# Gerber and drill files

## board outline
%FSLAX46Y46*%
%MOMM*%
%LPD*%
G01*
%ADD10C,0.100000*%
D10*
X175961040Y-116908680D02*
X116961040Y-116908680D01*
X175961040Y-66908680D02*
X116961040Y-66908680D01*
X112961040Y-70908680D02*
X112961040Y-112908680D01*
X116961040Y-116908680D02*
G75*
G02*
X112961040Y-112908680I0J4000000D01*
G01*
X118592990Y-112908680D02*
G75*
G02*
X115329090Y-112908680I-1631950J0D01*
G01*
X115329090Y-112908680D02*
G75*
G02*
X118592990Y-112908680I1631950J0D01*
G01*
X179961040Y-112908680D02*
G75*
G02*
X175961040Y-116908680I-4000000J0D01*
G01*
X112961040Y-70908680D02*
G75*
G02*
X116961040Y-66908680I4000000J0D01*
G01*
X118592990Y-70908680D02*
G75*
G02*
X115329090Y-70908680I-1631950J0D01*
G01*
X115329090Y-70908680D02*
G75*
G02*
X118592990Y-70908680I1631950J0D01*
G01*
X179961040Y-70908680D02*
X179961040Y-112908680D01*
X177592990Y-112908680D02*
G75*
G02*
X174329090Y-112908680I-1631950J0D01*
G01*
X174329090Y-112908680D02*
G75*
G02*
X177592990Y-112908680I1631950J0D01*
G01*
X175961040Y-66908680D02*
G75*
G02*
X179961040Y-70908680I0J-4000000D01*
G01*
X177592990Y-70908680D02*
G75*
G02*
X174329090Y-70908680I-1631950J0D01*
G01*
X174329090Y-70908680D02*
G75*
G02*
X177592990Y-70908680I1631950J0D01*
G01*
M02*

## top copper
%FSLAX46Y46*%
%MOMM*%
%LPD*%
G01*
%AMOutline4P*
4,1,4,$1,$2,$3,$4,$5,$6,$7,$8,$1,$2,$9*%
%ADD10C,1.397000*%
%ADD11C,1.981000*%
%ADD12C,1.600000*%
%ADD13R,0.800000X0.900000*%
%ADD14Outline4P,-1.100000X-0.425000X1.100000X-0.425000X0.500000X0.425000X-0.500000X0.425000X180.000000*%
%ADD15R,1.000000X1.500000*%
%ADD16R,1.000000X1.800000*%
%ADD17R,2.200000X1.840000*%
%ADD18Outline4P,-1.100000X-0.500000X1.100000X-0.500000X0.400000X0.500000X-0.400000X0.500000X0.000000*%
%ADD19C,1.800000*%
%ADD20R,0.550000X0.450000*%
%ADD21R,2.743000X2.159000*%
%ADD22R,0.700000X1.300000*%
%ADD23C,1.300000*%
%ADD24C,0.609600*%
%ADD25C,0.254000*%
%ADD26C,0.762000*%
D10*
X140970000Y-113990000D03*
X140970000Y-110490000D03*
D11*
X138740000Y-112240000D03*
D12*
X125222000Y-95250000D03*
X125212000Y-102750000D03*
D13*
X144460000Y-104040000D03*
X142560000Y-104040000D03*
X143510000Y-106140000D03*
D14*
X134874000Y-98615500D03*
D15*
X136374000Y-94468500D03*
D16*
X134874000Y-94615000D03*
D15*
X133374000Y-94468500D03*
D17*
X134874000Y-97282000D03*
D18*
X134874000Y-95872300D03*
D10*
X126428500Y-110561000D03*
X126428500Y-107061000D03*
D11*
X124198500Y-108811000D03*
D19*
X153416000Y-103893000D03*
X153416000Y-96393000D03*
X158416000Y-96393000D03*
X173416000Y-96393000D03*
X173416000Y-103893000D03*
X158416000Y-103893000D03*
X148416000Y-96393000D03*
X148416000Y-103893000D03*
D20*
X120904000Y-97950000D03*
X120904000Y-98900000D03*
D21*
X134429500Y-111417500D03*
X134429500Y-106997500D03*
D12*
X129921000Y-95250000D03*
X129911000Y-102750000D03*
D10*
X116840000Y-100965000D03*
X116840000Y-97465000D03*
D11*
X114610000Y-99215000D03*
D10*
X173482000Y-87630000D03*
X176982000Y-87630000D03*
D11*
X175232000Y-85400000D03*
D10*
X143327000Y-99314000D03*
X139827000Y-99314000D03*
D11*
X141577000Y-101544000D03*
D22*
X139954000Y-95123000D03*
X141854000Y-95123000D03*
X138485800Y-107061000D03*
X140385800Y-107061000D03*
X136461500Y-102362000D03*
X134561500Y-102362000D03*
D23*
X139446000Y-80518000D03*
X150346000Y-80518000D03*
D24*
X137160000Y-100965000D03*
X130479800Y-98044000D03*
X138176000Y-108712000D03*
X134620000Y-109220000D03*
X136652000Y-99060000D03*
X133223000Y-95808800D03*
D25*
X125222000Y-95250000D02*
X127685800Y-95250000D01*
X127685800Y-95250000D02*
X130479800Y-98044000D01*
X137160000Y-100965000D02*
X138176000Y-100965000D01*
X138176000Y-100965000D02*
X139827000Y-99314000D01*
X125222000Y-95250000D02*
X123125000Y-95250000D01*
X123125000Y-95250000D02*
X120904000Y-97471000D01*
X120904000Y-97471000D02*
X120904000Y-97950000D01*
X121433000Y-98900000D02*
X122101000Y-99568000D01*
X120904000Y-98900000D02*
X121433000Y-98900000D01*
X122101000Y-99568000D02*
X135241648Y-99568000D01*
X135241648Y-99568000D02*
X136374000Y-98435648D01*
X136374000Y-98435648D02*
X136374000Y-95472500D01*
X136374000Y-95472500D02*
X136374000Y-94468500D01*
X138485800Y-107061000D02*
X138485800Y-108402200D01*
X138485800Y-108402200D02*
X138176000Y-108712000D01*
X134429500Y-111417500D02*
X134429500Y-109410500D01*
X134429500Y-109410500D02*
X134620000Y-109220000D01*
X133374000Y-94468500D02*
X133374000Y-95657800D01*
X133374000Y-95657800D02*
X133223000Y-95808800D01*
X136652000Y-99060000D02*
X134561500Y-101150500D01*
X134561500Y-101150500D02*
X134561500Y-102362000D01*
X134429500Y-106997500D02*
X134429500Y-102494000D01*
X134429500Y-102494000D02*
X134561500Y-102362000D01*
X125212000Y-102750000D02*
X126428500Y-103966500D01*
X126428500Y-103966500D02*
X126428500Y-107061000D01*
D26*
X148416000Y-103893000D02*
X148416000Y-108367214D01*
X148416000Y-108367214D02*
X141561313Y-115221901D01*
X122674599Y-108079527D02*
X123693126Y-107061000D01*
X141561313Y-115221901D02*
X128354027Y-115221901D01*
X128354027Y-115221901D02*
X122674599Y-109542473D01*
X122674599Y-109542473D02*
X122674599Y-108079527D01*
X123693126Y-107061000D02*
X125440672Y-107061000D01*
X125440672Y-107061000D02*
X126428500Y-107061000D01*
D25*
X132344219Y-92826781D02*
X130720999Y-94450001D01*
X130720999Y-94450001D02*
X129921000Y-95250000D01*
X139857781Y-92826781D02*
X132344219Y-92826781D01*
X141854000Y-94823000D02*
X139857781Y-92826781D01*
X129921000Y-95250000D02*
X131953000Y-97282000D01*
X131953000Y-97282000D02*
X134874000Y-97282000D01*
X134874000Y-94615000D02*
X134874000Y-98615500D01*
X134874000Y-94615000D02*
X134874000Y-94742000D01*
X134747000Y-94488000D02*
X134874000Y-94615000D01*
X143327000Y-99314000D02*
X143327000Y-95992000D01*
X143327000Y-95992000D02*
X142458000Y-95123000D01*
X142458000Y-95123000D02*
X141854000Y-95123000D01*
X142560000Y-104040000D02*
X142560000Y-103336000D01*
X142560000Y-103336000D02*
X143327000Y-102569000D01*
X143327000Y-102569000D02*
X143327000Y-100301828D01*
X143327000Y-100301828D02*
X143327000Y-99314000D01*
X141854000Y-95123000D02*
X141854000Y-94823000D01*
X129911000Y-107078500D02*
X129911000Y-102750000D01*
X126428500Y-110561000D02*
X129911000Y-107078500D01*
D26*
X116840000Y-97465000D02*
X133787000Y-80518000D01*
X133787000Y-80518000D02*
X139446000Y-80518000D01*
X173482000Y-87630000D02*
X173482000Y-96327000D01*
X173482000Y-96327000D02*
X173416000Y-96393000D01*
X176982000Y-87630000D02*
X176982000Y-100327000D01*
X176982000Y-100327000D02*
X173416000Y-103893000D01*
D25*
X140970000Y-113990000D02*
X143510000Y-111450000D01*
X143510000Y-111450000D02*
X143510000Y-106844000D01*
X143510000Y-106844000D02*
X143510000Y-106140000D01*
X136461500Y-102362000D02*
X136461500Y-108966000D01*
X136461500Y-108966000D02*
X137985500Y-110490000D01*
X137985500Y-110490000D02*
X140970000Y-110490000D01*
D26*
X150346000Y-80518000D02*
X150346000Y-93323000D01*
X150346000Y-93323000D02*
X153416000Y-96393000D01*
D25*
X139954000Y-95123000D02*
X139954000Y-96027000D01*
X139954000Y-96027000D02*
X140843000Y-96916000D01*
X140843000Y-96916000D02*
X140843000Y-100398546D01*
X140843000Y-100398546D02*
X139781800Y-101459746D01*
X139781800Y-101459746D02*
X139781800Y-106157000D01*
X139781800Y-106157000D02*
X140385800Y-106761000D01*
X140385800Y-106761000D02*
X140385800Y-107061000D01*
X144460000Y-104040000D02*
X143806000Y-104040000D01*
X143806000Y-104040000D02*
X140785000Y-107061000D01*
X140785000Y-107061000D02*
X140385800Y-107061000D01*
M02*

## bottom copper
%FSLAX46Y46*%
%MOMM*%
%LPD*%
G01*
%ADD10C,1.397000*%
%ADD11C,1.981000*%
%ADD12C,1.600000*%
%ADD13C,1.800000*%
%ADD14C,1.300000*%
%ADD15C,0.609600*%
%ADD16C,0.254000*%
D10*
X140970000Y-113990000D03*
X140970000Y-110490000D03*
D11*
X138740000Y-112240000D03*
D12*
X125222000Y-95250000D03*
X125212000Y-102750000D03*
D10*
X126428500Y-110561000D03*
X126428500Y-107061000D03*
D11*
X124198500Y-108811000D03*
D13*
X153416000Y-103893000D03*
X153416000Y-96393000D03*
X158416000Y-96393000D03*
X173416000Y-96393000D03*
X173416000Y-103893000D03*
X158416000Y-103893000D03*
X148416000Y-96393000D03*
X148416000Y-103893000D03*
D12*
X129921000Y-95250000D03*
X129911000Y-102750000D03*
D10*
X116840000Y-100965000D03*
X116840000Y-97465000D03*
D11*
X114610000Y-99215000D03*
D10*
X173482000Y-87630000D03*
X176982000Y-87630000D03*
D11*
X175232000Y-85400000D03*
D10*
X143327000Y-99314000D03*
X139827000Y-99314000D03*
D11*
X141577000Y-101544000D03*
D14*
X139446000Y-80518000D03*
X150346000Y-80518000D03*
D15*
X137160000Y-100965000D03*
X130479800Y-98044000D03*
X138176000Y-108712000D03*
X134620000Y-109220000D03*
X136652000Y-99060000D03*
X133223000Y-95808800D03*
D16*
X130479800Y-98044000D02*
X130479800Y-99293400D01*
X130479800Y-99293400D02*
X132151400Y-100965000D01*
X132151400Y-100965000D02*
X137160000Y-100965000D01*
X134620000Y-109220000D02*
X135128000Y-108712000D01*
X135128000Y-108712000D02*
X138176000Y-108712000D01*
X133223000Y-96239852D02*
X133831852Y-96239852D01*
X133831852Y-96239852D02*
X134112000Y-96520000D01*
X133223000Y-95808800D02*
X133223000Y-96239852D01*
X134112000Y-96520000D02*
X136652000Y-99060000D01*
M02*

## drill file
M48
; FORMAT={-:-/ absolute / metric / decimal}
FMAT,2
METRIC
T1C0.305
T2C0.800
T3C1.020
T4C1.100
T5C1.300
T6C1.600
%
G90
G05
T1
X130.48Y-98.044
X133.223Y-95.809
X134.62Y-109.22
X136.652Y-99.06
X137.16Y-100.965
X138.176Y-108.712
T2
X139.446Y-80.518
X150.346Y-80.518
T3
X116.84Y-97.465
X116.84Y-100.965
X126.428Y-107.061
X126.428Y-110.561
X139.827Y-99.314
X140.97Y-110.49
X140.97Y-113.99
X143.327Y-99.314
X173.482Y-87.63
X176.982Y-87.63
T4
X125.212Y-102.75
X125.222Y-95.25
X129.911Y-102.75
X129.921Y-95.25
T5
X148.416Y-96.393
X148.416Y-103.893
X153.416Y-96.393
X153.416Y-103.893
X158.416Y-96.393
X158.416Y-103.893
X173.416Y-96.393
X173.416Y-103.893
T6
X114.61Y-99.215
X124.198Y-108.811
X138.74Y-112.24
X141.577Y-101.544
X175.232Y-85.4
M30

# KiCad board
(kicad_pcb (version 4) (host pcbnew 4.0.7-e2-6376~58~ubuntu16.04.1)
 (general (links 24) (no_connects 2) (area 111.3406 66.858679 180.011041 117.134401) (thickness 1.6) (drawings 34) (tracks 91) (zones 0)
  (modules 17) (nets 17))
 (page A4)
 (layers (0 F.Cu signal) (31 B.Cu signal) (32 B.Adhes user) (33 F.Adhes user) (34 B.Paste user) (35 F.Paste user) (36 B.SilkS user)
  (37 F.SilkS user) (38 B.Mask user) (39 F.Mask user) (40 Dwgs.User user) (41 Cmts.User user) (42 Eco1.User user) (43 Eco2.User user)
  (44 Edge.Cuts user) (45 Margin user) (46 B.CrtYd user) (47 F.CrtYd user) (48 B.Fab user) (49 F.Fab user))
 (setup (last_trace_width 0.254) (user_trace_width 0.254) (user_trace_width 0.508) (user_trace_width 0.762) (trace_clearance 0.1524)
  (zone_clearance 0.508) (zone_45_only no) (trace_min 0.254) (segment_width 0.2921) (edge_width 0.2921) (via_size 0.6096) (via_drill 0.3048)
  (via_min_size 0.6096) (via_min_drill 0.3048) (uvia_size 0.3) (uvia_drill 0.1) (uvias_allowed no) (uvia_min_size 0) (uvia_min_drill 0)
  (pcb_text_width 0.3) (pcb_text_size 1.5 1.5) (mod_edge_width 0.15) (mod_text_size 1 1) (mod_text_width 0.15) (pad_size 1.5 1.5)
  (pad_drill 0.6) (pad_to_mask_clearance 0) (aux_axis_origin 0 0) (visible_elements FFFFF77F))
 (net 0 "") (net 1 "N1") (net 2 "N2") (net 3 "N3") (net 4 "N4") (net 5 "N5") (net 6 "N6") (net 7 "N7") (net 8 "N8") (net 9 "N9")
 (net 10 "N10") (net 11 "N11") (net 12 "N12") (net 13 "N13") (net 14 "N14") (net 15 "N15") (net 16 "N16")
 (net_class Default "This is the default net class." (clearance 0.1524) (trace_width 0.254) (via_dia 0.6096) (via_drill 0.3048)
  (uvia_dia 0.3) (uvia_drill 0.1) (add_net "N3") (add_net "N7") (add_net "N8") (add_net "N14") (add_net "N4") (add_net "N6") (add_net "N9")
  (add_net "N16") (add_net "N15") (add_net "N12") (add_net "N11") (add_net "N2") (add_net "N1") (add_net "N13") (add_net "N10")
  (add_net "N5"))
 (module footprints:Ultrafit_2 (layer F.Cu) (at 140.97 113.99 180)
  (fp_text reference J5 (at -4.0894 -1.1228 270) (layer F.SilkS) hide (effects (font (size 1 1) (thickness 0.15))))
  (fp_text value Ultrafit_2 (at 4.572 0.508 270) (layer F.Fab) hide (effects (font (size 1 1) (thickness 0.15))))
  (pad 2 thru_hole circle (at 0 0 180) (size 1.397 1.397) (drill 1.02) (layers *.Cu *.Mask) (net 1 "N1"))
  (pad 1 thru_hole circle (at 0 3.5 180) (size 1.397 1.397) (drill 1.02) (layers *.Cu *.Mask) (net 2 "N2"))
  (pad "" thru_hole circle (at 2.23 1.75 180) (size 1.981 1.981) (drill 1.6) (layers *.Cu *.Mask)))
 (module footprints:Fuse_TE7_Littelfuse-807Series (layer F.Cu) (at 125.222 95.25 270)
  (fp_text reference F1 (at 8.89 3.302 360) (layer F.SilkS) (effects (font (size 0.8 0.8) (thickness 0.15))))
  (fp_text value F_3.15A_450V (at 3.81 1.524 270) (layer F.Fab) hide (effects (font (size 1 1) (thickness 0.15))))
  (pad 1 thru_hole circle (at 0 0 270) (size 1.6 1.6) (drill 1.1) (layers *.Cu *.Mask) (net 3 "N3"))
  (pad 2 thru_hole circle (at 7.5 0.01 270) (size 1.6 1.6) (drill 1.1) (layers *.Cu *.Mask) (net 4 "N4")))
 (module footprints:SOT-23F (layer F.Cu) (at 143.51 105.09 270)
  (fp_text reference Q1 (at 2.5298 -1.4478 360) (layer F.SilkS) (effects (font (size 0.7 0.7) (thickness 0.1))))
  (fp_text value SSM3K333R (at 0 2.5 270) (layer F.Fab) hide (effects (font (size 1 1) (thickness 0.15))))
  (pad 1 smd rect (at -1.05 -0.95 270) (size 0.9 0.8) (layers F.Cu F.Paste F.Mask) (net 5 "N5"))
  (pad 2 smd rect (at -1.05 0.95 270) (size 0.9 0.8) (layers F.Cu F.Paste F.Mask) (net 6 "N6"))
  (pad 3 smd rect (at 1.05 0 270) (size 0.9 0.8) (layers F.Cu F.Paste F.Mask) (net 1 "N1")))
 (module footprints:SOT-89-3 (layer F.Cu) (at 134.874 95.9485 270)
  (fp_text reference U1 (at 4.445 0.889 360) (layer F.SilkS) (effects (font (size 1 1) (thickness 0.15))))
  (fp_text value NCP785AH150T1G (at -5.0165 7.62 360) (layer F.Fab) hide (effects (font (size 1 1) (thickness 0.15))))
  (pad 2 smd trapezoid (at 2.667 0 180) (size 1.6 0.85) (rect_delta 0 0.6) (layers F.Cu F.Paste F.Mask) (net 6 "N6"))
  (pad 1 smd rect (at -1.48 -1.5 180) (size 1 1.5) (layers F.Cu F.Paste F.Mask) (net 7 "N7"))
  (pad 2 smd rect (at -1.3335 0 180) (size 1 1.8) (layers F.Cu F.Paste F.Mask) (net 6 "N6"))
  (pad 3 smd rect (at -1.48 1.5 180) (size 1 1.5) (layers F.Cu F.Paste F.Mask) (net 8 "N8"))
  (pad 2 smd rect (at 1.3335 0 180) (size 2.2 1.84) (layers F.Cu F.Paste F.Mask) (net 6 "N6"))
  (pad 2 smd trapezoid (at -0.0762 0) (size 1.5 1) (rect_delta 0 0.7) (layers F.Cu F.Paste F.Mask) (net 6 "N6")))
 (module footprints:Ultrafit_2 (layer F.Cu) (at 126.4285 110.561 180)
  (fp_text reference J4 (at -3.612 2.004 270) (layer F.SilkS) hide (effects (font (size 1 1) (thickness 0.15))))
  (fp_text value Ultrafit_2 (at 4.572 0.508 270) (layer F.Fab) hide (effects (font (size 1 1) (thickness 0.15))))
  (pad 2 thru_hole circle (at 0 0 180) (size 1.397 1.397) (drill 1.02) (layers *.Cu *.Mask) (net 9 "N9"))
  (pad 1 thru_hole circle (at 0 3.5 180) (size 1.397 1.397) (drill 1.02) (layers *.Cu *.Mask) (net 4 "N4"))
  (pad "" thru_hole circle (at 2.23 1.75 180) (size 1.981 1.981) (drill 1.6) (layers *.Cu *.Mask)))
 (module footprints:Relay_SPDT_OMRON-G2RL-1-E (layer F.Cu) (at 173.416 96.393 180)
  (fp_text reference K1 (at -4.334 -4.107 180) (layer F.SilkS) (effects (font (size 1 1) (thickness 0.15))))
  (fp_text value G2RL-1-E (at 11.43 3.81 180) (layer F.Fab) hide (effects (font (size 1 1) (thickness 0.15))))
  (pad 3 thru_hole circle (at 20 -7.5 180) (size 1.8 1.8) (drill 1.3) (layers *.Cu *.Mask))
  (pad 6 thru_hole circle (at 20 0 180) (size 1.8 1.8) (drill 1.3) (layers *.Cu *.Mask) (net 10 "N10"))
  (pad 7 thru_hole circle (at 15 0 180) (size 1.8 1.8) (drill 1.3) (layers *.Cu *.Mask))
  (pad 8 thru_hole circle (at 0 0 180) (size 1.8 1.8) (drill 1.3) (layers *.Cu *.Mask) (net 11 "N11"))
  (pad 1 thru_hole circle (at 0 -7.5 180) (size 1.8 1.8) (drill 1.3) (layers *.Cu *.Mask) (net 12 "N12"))
  (pad 2 thru_hole circle (at 15 -7.5 180) (size 1.8 1.8) (drill 1.3) (layers *.Cu *.Mask) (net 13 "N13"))
  (pad 5 thru_hole circle (at 25 0 180) (size 1.8 1.8) (drill 1.3) (layers *.Cu *.Mask))
  (pad 4 thru_hole circle (at 25 -7.5 180) (size 1.8 1.8) (drill 1.3) (layers *.Cu *.Mask) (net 4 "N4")))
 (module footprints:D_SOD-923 (layer F.Cu) (at 120.904 98.425 270)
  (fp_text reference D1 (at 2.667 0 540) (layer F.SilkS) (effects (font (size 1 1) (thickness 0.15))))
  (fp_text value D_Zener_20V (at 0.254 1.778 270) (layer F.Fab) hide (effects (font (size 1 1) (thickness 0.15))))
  (pad 1 smd rect (at -0.475 0 270) (size 0.45 0.55) (layers F.Cu F.Paste F.Mask) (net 3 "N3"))
  (pad 2 smd rect (at 0.475 0 270) (size 0.45 0.55) (layers F.Cu F.Paste F.Mask) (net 7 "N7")))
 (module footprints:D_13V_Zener (layer F.Cu) (at 134.4295 109.2075 270)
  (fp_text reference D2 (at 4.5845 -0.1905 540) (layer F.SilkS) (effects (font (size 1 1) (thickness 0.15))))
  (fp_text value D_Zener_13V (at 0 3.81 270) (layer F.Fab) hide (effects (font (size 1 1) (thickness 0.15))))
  (pad 2 smd rect (at 2.21 0 90) (size 2.159 2.743) (layers F.Cu F.Paste F.Mask) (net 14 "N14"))
  (pad 1 smd rect (at -2.21 0 90) (size 2.159 2.743) (layers F.Cu F.Paste F.Mask) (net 8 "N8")))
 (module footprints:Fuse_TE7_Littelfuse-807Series (layer F.Cu) (at 129.921 95.25 270)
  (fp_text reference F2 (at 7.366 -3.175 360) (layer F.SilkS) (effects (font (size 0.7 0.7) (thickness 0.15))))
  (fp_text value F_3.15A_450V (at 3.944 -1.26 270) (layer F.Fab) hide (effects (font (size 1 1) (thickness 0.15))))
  (pad 1 thru_hole circle (at 0 0 270) (size 1.6 1.6) (drill 1.1) (layers *.Cu *.Mask) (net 6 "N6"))
  (pad 2 thru_hole circle (at 7.5 0.01 270) (size 1.6 1.6) (drill 1.1) (layers *.Cu *.Mask) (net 9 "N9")))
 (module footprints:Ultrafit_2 (layer F.Cu) (at 116.84 100.965 180)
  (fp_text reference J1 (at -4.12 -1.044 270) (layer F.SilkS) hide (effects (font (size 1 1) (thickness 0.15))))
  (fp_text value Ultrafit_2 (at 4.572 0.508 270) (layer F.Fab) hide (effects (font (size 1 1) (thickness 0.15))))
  (pad 2 thru_hole circle (at 0 0 180) (size 1.397 1.397) (drill 1.02) (layers *.Cu *.Mask) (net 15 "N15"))
  (pad 1 thru_hole circle (at 0 3.5 180) (size 1.397 1.397) (drill 1.02) (layers *.Cu *.Mask) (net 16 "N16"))
  (pad "" thru_hole circle (at 2.23 1.75 180) (size 1.981 1.981) (drill 1.6) (layers *.Cu *.Mask)))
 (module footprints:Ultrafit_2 (layer F.Cu) (at 173.482 87.63 90)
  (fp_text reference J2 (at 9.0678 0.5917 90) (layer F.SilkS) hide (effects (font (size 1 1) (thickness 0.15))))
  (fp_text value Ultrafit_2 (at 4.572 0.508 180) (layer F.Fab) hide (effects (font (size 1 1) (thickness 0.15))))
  (pad 2 thru_hole circle (at 0 0 90) (size 1.397 1.397) (drill 1.02) (layers *.Cu *.Mask) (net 11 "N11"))
  (pad 1 thru_hole circle (at 0 3.5 90) (size 1.397 1.397) (drill 1.02) (layers *.Cu *.Mask) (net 12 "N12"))
  (pad "" thru_hole circle (at 2.23 1.75 90) (size 1.981 1.981) (drill 1.6) (layers *.Cu *.Mask)))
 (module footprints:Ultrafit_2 (layer F.Cu) (at 143.327 99.314 270)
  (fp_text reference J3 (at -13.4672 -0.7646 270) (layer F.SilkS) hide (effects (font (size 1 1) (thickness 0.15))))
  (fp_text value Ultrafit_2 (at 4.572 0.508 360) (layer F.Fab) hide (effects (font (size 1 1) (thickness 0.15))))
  (pad 2 thru_hole circle (at 0 0 270) (size 1.397 1.397) (drill 1.02) (layers *.Cu *.Mask) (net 6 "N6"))
  (pad 1 thru_hole circle (at 0 3.5 270) (size 1.397 1.397) (drill 1.02) (layers *.Cu *.Mask) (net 3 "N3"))
  (pad "" thru_hole circle (at 2.23 1.75 270) (size 1.981 1.981) (drill 1.6) (layers *.Cu *.Mask)))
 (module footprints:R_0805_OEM (layer F.Cu) (at 140.904 95.123)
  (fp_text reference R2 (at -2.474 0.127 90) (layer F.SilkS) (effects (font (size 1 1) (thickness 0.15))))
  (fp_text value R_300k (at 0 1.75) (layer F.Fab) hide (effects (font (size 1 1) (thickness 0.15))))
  (pad 1 smd rect (at -0.95 0) (size 0.7 1.3) (layers F.Cu F.Paste F.Mask) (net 5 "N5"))
  (pad 2 smd rect (at 0.95 0) (size 0.7 1.3) (layers F.Cu F.Paste F.Mask) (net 6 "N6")))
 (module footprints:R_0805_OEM (layer F.Cu) (at 139.4358 107.061)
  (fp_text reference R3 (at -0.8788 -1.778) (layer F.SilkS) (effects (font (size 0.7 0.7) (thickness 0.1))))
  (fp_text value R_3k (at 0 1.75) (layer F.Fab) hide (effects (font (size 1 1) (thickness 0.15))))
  (pad 1 smd rect (at -0.95 0) (size 0.7 1.3) (layers F.Cu F.Paste F.Mask) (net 14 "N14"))
  (pad 2 smd rect (at 0.95 0) (size 0.7 1.3) (layers F.Cu F.Paste F.Mask) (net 5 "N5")))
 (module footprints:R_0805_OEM (layer F.Cu) (at 135.5115 102.362 180)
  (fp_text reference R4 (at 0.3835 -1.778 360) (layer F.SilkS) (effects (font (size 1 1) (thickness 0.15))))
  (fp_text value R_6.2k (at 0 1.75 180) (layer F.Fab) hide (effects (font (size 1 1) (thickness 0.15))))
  (pad 1 smd rect (at -0.95 0 180) (size 0.7 1.3) (layers F.Cu F.Paste F.Mask) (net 2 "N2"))
  (pad 2 smd rect (at 0.95 0 180) (size 0.7 1.3) (layers F.Cu F.Paste F.Mask) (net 8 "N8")))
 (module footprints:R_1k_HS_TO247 (layer F.Cu) (at 139.446 80.518)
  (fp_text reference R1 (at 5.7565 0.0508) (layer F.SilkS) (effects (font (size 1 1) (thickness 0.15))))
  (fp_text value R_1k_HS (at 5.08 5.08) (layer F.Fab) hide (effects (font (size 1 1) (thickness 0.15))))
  (pad 1 thru_hole circle (at 0 0) (size 1.3 1.3) (drill 0.8) (layers *.Cu *.Mask) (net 16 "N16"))
  (pad 2 thru_hole circle (at 10.9 0) (size 1.3 1.3) (drill 0.8) (layers *.Cu *.Mask) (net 10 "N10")))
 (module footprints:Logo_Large (layer B.Cu) (at 144.5895 73.2409 180)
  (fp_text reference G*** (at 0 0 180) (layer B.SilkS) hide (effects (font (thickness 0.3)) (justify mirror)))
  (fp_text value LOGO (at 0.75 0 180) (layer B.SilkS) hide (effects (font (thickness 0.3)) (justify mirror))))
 (gr_line (start 175.96104 116.90868) (end 116.96104 116.90868) (layer Edge.Cuts) (width 0.1))
 (gr_line (start 175.96104 66.90868) (end 116.96104 66.90868) (layer Edge.Cuts) (width 0.1))
 (gr_line (start 112.96104 70.90868) (end 112.96104 112.90868) (layer Edge.Cuts) (width 0.1))
 (gr_arc (start 116.96104 112.90868) (end 112.96104 112.90868) (angle -90) (layer Edge.Cuts) (width 0.1))
 (gr_circle (center 116.96104 112.90868) (end 118.59299 112.90868) (layer Edge.Cuts) (width 0.1))
 (gr_arc (start 175.96104 112.90868) (end 175.96104 116.90868) (angle -90) (layer Edge.Cuts) (width 0.1))
 (gr_arc (start 116.96104 70.90868) (end 116.96104 66.90868) (angle -90) (layer Edge.Cuts) (width 0.1))
 (gr_circle (center 116.96104 70.90868) (end 118.59299 70.90868) (layer Edge.Cuts) (width 0.1))
 (gr_line (start 179.96104 70.90868) (end 179.96104 112.90868) (layer Edge.Cuts) (width 0.1))
 (gr_circle (center 175.96104 112.90868) (end 177.59299 112.90868) (layer Edge.Cuts) (width 0.1))
 (gr_arc (start 175.96104 70.90868) (end 179.96104 70.90868) (angle -90) (layer Edge.Cuts) (width 0.1))
 (gr_circle (center 175.96104 70.90868) (end 177.59299 70.90868) (layer Edge.Cuts) (width 0.1))
 (segment (start 130.4798 98.044) (end 130.4798 99.2934) (width 0.254) (layer B.Cu) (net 3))
 (segment (start 130.4798 99.2934) (end 132.1514 100.965) (width 0.254) (layer B.Cu) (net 3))
 (segment (start 125.222 95.25) (end 127.6858 95.25) (width 0.254) (layer F.Cu) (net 3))
 (segment (start 127.6858 95.25) (end 130.4798 98.044) (width 0.254) (layer F.Cu) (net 3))
 (segment (start 137.16 100.965) (end 138.176 100.965) (width 0.254) (layer F.Cu) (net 3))
 (segment (start 138.176 100.965) (end 139.827 99.314) (width 0.254) (layer F.Cu) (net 3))
 (segment (start 132.1514 100.965) (end 137.16 100.965) (width 0.254) (layer B.Cu) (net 3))
 (via (at 137.16 100.965) (size 0.6096) (drill 0.3048) (layers F.Cu B.Cu) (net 3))
 (via (at 130.4798 98.044) (size 0.6096) (drill 0.3048) (layers F.Cu B.Cu) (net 3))
 (segment (start 125.222 95.25) (end 123.125 95.25) (width 0.254) (layer F.Cu) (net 3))
 (segment (start 123.125 95.25) (end 120.904 97.471) (width 0.254) (layer F.Cu) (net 3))
 (segment (start 120.904 97.471) (end 120.904 97.95) (width 0.254) (layer F.Cu) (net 3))
 (segment (start 121.433 98.9) (end 122.101 99.568) (width 0.254) (layer F.Cu) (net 7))
 (segment (start 120.904 98.9) (end 121.433 98.9) (width 0.254) (layer F.Cu) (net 7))
 (segment (start 122.101 99.568) (end 135.241648 99.568) (width 0.254) (layer F.Cu) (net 7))
 (segment (start 135.241648 99.568) (end 136.374 98.435648) (width 0.254) (layer F.Cu) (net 7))
 (segment (start 136.374 98.435648) (end 136.374 95.4725) (width 0.254) (layer F.Cu) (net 7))
 (segment (start 136.374 95.4725) (end 136.374 94.4685) (width 0.254) (layer F.Cu) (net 7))
 (segment (start 138.4858 107.061) (end 138.4858 108.4022) (width 0.254) (layer F.Cu) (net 14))
 (segment (start 138.4858 108.4022) (end 138.176 108.712) (width 0.254) (layer F.Cu) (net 14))
 (segment (start 134.62 109.22) (end 135.128 108.712) (width 0.254) (layer B.Cu) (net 14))
 (segment (start 135.128 108.712) (end 138.176 108.712) (width 0.254) (layer B.Cu) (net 14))
 (via (at 138.176 108.712) (size 0.6096) (drill 0.3048) (layers F.Cu B.Cu) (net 14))
 (segment (start 134.4295 111.4175) (end 134.4295 109.4105) (width 0.254) (layer F.Cu) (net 14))
 (segment (start 134.4295 109.4105) (end 134.62 109.22) (width 0.254) (layer F.Cu) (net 14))
 (via (at 134.62 109.22) (size 0.6096) (drill 0.3048) (layers F.Cu B.Cu) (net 14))
 (segment (start 133.374 94.4685) (end 133.374 95.6578) (width 0.254) (layer F.Cu) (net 8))
 (segment (start 133.374 95.6578) (end 133.223 95.8088) (width 0.254) (layer F.Cu) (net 8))
 (segment (start 133.223 96.239852) (end 133.831852 96.239852) (width 0.254) (layer B.Cu) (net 8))
 (segment (start 133.831852 96.239852) (end 134.112 96.52) (width 0.254) (layer B.Cu) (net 8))
 (segment (start 133.223 95.8088) (end 133.223 96.239852) (width 0.254) (layer B.Cu) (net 8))
 (segment (start 136.652 99.06) (end 134.5615 101.1505) (width 0.254) (layer F.Cu) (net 8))
 (segment (start 134.5615 101.1505) (end 134.5615 102.362) (width 0.254) (layer F.Cu) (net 8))
 (via (at 136.652 99.06) (size 0.6096) (drill 0.3048) (layers F.Cu B.Cu) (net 8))
 (segment (start 134.112 96.52) (end 136.652 99.06) (width 0.254) (layer B.Cu) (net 8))
 (via (at 133.223 95.8088) (size 0.6096) (drill 0.3048) (layers F.Cu B.Cu) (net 8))
 (segment (start 134.4295 106.9975) (end 134.4295 102.494) (width 0.254) (layer F.Cu) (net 8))
 (segment (start 134.4295 102.494) (end 134.5615 102.362) (width 0.254) (layer F.Cu) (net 8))
 (segment (start 125.212 102.75) (end 126.4285 103.9665) (width 0.254) (layer F.Cu) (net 4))
 (segment (start 126.4285 103.9665) (end 126.4285 107.061) (width 0.254) (layer F.Cu) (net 4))
 (segment (start 148.416 103.893) (end 148.416 108.367214) (width 0.762) (layer F.Cu) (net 4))
 (segment (start 148.416 108.367214) (end 141.561313 115.221901) (width 0.762) (layer F.Cu) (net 4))
 (segment (start 122.674599 108.079527) (end 123.693126 107.061) (width 0.762) (layer F.Cu) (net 4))
 (segment (start 141.561313 115.221901) (end 128.354027 115.221901) (width 0.762) (layer F.Cu) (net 4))
 (segment (start 128.354027 115.221901) (end 122.674599 109.542473) (width 0.762) (layer F.Cu) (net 4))
 (segment (start 122.674599 109.542473) (end 122.674599 108.079527) (width 0.762) (layer F.Cu) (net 4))
 (segment (start 123.693126 107.061) (end 125.440672 107.061) (width 0.762) (layer F.Cu) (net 4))
 (segment (start 125.440672 107.061) (end 126.4285 107.061) (width 0.762) (layer F.Cu) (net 4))
 (segment (start 132.344219 92.826781) (end 130.720999 94.450001) (width 0.254) (layer F.Cu) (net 6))
 (segment (start 130.720999 94.450001) (end 129.921 95.25) (width 0.254) (layer F.Cu) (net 6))
 (segment (start 139.857781 92.826781) (end 132.344219 92.826781) (width 0.254) (layer F.Cu) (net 6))
 (segment (start 141.854 94.823) (end 139.857781 92.826781) (width 0.254) (layer F.Cu) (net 6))
 (segment (start 129.921 95.25) (end 131.953 97.282) (width 0.254) (layer F.Cu) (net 6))
 (segment (start 131.953 97.282) (end 134.874 97.282) (width 0.254) (layer F.Cu) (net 6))
 (segment (start 134.874 94.615) (end 134.874 98.6155) (width 0.254) (layer F.Cu) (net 6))
 (segment (start 134.874 94.615) (end 134.874 94.742) (width 0.254) (layer F.Cu) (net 6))
 (segment (start 134.747 94.488) (end 134.874 94.615) (width 0.254) (layer F.Cu) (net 6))
 (segment (start 143.327 99.314) (end 143.327 95.992) (width 0.254) (layer F.Cu) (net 6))
 (segment (start 143.327 95.992) (end 142.458 95.123) (width 0.254) (layer F.Cu) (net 6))
 (segment (start 142.458 95.123) (end 141.854 95.123) (width 0.254) (layer F.Cu) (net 6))
 (segment (start 142.56 104.04) (end 142.56 103.336) (width 0.254) (layer F.Cu) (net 6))
 (segment (start 142.56 103.336) (end 143.327 102.569) (width 0.254) (layer F.Cu) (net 6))
 (segment (start 143.327 102.569) (end 143.327 100.301828) (width 0.254) (layer F.Cu) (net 6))
 (segment (start 143.327 100.301828) (end 143.327 99.314) (width 0.254) (layer F.Cu) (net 6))
 (segment (start 141.854 95.123) (end 141.854 94.823) (width 0.254) (layer F.Cu) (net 6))
 (segment (start 129.911 107.0785) (end 129.911 102.75) (width 0.254) (layer F.Cu) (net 9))
 (segment (start 126.4285 110.561) (end 129.911 107.0785) (width 0.254) (layer F.Cu) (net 9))
 (segment (start 116.84 97.465) (end 133.787 80.518) (width 0.762) (layer F.Cu) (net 16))
 (segment (start 133.787 80.518) (end 139.446 80.518) (width 0.762) (layer F.Cu) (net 16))
 (segment (start 173.482 87.63) (end 173.482 96.327) (width 0.762) (layer F.Cu) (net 11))
 (segment (start 173.482 96.327) (end 173.416 96.393) (width 0.762) (layer F.Cu) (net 11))
 (segment (start 176.982 87.63) (end 176.982 100.327) (width 0.762) (layer F.Cu) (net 12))
 (segment (start 176.982 100.327) (end 173.416 103.893) (width 0.762) (layer F.Cu) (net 12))
 (segment (start 140.97 113.99) (end 143.51 111.45) (width 0.254) (layer F.Cu) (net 1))
 (segment (start 143.51 111.45) (end 143.51 106.844) (width 0.254) (layer F.Cu) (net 1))
 (segment (start 143.51 106.844) (end 143.51 106.14) (width 0.254) (layer F.Cu) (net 1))
 (segment (start 136.4615 102.362) (end 136.4615 108.966) (width 0.254) (layer F.Cu) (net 2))
 (segment (start 136.4615 108.966) (end 137.9855 110.49) (width 0.254) (layer F.Cu) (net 2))
 (segment (start 137.9855 110.49) (end 140.97 110.49) (width 0.254) (layer F.Cu) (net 2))
 (segment (start 150.346 80.518) (end 150.346 93.323) (width 0.762) (layer F.Cu) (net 10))
 (segment (start 150.346 93.323) (end 153.416 96.393) (width 0.762) (layer F.Cu) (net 10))
 (segment (start 139.954 95.123) (end 139.954 96.027) (width 0.254) (layer F.Cu) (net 5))
 (segment (start 139.954 96.027) (end 140.843 96.916) (width 0.254) (layer F.Cu) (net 5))
 (segment (start 140.843 96.916) (end 140.843 100.398546) (width 0.254) (layer F.Cu) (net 5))
 (segment (start 140.843 100.398546) (end 139.7818 101.459746) (width 0.254) (layer F.Cu) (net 5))
 (segment (start 139.7818 101.459746) (end 139.7818 106.157) (width 0.254) (layer F.Cu) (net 5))
 (segment (start 139.7818 106.157) (end 140.3858 106.761) (width 0.254) (layer F.Cu) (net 5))
 (segment (start 140.3858 106.761) (end 140.3858 107.061) (width 0.254) (layer F.Cu) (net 5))
 (segment (start 144.46 104.04) (end 143.806 104.04) (width 0.254) (layer F.Cu) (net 5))
 (segment (start 143.806 104.04) (end 140.785 107.061) (width 0.254) (layer F.Cu) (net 5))
 (segment (start 140.785 107.061) (end 140.3858 107.061) (width 0.254) (layer F.Cu) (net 5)))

